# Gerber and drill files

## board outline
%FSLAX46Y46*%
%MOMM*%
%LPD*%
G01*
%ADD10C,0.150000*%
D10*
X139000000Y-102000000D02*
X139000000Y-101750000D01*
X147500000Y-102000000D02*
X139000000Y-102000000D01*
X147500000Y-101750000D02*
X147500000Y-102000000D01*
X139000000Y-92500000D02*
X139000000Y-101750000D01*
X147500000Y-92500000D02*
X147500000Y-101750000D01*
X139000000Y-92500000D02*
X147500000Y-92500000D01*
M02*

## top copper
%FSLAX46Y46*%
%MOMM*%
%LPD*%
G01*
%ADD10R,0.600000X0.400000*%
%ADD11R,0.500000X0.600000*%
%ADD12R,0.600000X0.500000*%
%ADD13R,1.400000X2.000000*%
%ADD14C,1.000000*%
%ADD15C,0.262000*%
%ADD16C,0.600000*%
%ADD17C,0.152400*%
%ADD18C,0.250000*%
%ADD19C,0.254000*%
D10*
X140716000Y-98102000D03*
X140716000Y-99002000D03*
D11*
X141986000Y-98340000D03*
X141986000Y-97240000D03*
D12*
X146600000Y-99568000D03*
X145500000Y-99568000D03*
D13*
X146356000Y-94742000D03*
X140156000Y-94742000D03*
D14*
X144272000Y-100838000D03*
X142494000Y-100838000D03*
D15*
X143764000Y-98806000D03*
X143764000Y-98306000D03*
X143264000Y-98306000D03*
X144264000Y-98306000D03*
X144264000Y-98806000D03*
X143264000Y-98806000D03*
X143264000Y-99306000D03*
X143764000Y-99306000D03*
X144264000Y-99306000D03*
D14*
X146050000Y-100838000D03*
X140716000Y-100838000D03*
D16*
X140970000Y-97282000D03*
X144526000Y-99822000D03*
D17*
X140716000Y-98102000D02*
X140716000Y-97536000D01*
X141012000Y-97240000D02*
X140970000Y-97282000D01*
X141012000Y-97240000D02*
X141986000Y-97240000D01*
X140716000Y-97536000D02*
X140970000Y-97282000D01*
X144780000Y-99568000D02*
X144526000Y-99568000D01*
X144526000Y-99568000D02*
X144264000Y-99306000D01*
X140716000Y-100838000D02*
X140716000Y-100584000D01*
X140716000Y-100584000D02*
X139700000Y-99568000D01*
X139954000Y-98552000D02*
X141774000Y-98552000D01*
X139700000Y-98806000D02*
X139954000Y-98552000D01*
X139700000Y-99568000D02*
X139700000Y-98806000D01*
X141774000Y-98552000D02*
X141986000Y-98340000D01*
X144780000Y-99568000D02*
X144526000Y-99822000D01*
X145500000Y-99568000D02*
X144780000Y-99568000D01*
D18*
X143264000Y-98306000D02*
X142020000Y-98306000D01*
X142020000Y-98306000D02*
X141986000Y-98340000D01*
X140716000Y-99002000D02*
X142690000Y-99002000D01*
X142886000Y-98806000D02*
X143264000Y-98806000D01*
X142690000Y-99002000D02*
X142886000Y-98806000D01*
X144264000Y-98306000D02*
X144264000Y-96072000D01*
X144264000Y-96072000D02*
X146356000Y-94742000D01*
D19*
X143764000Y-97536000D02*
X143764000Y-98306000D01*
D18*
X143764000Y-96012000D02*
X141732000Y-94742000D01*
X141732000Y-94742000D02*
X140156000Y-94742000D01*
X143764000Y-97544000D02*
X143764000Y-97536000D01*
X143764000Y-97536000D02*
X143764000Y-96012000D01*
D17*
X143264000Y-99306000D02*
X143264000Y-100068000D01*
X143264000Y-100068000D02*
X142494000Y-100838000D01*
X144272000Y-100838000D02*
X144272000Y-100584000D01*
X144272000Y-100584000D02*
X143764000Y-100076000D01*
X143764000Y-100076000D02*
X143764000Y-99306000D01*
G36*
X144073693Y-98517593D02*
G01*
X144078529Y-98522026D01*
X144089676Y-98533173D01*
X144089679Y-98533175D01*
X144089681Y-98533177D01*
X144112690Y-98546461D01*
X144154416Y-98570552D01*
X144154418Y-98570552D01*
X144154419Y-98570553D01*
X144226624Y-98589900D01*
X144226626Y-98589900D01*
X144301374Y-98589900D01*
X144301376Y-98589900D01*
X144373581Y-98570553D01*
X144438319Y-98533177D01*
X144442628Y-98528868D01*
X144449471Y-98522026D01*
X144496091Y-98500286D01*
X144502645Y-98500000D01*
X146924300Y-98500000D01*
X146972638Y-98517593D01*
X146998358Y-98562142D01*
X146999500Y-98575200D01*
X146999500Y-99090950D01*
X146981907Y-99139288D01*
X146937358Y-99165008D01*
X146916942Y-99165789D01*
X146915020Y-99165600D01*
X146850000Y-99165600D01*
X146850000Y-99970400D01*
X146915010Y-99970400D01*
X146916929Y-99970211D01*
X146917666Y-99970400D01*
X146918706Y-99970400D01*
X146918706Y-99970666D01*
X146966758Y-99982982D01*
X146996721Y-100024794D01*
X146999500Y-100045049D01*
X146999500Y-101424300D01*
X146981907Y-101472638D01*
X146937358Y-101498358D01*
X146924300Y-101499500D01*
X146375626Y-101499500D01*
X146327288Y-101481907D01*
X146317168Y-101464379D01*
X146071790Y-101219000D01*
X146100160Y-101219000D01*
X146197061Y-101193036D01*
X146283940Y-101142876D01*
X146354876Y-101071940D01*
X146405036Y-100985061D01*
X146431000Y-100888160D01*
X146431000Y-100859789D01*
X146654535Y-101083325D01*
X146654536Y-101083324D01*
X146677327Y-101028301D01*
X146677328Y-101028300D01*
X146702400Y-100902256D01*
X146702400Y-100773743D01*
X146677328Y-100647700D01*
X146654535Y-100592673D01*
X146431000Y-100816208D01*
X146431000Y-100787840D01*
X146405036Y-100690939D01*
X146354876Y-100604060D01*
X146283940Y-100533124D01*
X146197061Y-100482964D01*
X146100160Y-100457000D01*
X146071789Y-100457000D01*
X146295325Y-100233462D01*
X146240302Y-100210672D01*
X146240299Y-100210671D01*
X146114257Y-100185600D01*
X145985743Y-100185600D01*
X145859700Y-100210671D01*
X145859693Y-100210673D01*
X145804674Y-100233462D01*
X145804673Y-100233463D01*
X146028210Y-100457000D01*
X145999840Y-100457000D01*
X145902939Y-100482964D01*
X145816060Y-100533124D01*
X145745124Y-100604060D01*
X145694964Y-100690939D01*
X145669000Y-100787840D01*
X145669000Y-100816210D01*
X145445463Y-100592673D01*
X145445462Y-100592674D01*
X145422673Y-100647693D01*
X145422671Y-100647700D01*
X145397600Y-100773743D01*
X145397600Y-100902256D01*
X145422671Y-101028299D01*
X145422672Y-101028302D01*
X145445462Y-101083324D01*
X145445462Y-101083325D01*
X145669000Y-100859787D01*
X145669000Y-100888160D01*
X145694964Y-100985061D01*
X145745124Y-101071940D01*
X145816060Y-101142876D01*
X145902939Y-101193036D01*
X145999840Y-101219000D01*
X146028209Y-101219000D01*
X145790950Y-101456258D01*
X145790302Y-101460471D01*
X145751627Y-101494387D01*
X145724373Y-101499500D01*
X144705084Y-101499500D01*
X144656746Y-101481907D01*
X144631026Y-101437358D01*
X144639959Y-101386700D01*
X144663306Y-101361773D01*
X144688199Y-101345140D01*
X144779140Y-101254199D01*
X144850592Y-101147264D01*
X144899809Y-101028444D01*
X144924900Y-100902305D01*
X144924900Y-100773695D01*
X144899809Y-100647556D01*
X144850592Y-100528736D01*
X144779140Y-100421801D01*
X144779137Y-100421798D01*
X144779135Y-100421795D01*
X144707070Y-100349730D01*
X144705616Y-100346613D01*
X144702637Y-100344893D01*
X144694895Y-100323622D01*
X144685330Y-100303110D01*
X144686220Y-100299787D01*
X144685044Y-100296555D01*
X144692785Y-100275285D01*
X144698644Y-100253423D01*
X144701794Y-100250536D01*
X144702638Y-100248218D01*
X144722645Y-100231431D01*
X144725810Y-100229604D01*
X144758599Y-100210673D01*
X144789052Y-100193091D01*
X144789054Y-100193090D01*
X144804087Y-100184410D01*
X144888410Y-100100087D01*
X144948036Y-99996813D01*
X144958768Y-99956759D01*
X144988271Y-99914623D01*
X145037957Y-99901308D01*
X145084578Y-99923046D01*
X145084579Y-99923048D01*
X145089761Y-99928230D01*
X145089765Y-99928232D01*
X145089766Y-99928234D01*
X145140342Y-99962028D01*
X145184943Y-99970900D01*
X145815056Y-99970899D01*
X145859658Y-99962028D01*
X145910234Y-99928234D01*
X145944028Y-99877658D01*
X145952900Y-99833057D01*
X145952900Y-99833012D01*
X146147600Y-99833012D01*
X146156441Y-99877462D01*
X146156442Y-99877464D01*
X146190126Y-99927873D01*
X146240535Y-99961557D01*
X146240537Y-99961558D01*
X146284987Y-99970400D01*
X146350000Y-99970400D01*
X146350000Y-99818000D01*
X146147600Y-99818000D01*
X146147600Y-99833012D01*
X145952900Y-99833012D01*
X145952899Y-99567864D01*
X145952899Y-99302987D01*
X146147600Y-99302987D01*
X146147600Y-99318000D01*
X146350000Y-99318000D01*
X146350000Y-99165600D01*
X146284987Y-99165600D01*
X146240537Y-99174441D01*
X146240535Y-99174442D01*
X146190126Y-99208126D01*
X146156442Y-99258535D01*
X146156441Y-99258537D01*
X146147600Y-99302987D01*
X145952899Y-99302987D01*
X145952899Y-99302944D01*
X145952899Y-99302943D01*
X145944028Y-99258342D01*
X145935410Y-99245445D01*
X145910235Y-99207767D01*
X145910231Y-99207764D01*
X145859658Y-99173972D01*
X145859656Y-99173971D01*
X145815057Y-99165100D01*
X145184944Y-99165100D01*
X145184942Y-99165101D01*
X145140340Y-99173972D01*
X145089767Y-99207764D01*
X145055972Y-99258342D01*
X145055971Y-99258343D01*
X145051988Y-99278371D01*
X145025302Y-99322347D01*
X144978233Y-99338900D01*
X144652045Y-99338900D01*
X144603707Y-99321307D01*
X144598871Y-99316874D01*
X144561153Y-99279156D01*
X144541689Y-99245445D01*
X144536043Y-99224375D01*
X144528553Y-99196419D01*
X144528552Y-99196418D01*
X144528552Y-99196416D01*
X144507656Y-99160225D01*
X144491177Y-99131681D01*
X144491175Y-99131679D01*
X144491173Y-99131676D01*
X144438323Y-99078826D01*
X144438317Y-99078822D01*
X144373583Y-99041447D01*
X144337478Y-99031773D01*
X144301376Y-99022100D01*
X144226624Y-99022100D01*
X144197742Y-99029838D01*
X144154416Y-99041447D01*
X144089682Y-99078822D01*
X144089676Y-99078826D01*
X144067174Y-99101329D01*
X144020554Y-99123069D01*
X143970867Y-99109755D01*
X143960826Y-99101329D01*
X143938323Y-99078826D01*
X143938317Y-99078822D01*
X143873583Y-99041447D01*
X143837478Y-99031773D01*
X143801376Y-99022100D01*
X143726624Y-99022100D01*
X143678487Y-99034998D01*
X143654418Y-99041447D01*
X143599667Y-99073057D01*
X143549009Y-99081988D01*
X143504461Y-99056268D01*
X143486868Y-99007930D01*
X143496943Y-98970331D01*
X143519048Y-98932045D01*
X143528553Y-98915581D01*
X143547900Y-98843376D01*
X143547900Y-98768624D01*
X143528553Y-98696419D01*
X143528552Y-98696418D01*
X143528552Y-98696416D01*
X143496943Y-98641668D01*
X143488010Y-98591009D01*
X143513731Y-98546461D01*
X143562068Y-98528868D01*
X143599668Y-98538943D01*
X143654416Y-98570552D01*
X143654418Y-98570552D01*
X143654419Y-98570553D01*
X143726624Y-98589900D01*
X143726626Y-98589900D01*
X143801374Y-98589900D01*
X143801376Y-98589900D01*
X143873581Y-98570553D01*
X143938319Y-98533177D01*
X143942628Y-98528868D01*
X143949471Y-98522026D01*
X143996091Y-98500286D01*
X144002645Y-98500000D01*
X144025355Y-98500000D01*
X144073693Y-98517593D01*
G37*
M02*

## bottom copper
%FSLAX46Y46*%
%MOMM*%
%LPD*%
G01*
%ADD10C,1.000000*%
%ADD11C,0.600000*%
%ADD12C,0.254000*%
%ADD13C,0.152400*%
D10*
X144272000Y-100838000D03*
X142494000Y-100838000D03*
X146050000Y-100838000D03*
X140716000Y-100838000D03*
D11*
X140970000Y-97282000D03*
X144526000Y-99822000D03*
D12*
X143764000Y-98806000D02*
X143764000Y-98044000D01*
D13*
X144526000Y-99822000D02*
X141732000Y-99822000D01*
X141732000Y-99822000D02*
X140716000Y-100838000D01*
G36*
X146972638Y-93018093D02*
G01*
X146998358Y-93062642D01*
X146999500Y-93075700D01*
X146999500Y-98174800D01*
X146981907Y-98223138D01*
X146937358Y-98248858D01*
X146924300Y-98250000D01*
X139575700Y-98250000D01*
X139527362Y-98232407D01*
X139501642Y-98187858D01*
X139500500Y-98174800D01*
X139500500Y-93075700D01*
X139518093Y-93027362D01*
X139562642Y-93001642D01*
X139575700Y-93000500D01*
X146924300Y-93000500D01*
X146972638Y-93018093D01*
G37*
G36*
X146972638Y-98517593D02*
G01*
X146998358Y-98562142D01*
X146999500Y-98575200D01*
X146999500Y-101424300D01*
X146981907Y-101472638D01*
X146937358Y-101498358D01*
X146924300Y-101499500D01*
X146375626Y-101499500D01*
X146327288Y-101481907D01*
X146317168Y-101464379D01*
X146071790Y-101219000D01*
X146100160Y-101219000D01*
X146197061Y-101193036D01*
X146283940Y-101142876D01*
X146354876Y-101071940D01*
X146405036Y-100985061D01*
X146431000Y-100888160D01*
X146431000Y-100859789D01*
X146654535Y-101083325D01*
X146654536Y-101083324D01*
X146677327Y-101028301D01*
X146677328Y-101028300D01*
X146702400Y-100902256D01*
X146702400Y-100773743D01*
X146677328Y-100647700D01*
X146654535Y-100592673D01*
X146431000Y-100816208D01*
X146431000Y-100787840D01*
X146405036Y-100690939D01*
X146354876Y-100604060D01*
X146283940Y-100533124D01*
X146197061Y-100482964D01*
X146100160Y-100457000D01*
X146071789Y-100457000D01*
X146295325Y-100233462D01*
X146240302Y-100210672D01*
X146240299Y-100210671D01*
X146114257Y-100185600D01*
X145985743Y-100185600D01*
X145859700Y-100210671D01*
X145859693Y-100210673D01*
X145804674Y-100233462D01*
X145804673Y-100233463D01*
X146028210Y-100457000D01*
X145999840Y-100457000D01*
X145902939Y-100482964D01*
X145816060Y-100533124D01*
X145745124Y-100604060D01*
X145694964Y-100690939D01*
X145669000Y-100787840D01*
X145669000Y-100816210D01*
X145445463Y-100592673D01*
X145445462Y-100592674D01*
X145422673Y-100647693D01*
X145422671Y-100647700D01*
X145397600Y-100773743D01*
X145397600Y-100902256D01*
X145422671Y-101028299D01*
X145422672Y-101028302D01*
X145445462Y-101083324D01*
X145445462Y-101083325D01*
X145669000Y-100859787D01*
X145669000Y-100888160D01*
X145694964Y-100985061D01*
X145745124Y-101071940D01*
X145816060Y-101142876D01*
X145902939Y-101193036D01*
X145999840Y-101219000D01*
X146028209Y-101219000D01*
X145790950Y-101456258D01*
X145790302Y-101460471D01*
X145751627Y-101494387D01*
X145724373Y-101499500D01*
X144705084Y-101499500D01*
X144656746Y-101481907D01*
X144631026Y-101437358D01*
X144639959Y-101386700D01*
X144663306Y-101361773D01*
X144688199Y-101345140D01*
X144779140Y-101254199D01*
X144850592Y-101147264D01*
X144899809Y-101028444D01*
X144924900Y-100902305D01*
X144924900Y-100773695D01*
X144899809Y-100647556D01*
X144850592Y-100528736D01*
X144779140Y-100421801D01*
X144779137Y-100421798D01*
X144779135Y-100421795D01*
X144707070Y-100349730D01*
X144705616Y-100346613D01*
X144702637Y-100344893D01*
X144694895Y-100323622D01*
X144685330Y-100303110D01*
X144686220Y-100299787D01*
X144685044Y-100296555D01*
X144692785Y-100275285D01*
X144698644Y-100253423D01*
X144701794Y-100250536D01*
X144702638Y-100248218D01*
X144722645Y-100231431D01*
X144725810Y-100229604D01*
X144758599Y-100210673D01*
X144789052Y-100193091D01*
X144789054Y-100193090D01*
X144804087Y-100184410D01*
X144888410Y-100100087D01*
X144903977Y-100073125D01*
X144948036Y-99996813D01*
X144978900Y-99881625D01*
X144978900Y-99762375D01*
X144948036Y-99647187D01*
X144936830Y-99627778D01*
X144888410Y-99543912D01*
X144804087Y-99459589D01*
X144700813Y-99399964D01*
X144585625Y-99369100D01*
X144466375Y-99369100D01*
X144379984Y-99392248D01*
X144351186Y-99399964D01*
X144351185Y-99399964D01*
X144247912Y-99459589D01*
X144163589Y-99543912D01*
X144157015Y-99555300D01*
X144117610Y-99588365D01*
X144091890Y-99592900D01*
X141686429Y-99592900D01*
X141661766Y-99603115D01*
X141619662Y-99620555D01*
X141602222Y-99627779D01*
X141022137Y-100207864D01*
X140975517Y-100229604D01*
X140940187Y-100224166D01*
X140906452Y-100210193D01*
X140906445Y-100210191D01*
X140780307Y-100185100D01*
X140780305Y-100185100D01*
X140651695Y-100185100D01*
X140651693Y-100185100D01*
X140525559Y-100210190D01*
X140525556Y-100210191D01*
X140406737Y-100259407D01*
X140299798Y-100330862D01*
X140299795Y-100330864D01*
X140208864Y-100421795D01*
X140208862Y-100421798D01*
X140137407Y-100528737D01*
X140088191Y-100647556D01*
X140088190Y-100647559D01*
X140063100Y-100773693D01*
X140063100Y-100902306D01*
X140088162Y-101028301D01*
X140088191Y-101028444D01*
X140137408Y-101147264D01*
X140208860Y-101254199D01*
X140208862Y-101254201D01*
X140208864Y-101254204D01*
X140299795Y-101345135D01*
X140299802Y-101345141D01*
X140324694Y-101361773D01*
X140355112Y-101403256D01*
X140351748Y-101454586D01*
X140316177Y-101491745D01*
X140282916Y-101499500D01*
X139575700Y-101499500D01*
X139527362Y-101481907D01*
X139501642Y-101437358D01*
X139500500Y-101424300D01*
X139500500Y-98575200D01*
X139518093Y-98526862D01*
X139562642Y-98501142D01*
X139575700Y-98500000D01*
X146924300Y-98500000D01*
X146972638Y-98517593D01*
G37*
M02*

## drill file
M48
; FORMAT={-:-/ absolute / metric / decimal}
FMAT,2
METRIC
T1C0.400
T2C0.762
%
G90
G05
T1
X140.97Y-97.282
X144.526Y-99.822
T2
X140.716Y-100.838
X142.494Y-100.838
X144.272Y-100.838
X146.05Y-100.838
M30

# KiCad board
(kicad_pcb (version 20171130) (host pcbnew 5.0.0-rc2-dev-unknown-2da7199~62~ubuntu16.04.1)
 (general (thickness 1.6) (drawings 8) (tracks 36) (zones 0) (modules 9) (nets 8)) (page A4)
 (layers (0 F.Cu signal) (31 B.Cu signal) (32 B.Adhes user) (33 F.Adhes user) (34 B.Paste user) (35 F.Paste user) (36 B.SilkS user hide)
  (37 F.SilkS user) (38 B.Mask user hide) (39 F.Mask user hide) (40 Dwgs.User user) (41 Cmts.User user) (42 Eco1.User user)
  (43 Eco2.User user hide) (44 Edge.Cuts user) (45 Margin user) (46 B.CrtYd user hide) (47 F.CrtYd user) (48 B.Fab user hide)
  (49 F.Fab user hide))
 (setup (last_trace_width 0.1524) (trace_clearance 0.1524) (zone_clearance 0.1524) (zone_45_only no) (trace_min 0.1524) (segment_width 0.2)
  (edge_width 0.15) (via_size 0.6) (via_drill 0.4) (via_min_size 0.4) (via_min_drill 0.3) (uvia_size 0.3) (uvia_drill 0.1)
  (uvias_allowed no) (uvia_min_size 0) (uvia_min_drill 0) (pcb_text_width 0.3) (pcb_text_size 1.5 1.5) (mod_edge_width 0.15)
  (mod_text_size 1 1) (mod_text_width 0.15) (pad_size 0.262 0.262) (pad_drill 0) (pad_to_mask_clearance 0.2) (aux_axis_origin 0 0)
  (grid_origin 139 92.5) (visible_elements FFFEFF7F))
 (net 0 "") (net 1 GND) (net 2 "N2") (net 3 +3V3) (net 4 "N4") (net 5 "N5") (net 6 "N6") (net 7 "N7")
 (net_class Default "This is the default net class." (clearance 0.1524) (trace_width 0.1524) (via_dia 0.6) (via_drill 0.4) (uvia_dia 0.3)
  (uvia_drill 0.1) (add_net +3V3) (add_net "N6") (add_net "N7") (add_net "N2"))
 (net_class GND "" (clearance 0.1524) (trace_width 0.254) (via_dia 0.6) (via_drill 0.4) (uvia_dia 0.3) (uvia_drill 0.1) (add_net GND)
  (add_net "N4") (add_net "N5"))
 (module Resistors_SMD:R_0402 (layer F.Cu) (at 140.716 98.552 270)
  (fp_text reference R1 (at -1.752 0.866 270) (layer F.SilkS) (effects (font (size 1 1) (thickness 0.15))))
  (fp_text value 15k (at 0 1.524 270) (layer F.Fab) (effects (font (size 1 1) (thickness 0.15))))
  (pad 1 smd rect (at -0.45 0 270) (size 0.4 0.6) (layers F.Cu F.Paste F.Mask) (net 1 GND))
  (pad 2 smd rect (at 0.45 0 270) (size 0.4 0.6) (layers F.Cu F.Paste F.Mask) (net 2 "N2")))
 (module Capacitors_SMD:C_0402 (layer F.Cu) (at 141.986 97.79 90)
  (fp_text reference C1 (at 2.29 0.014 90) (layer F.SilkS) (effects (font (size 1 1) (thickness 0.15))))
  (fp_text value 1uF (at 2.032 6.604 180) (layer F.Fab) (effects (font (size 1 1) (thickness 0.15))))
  (pad 1 smd rect (at -0.55 0 90) (size 0.6 0.5) (layers F.Cu F.Paste F.Mask) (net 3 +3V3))
  (pad 2 smd rect (at 0.55 0 90) (size 0.6 0.5) (layers F.Cu F.Paste F.Mask) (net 1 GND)))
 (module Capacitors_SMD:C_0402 (layer F.Cu) (at 146.05 99.568 180)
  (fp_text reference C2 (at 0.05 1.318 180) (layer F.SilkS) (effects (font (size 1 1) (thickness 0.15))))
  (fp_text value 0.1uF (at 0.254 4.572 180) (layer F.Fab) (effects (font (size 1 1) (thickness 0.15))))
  (pad 1 smd rect (at -0.55 0 180) (size 0.6 0.5) (layers F.Cu F.Paste F.Mask) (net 1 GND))
  (pad 2 smd rect (at 0.55 0 180) (size 0.6 0.5) (layers F.Cu F.Paste F.Mask) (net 3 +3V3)))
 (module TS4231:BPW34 (layer F.Cu) (at 143.256 94.742 180)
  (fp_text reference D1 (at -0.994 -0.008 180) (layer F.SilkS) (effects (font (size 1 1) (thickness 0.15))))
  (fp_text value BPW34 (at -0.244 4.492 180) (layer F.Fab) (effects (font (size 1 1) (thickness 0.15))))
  (pad 1 smd rect (at -3.1 0 180) (size 1.4 2) (layers F.Cu F.Paste F.Mask) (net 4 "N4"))
  (pad 2 smd rect (at 3.1 0 180) (size 1.4 2) (layers F.Cu F.Paste F.Mask) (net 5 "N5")))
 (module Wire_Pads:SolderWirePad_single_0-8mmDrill (layer F.Cu) (at 144.272 100.838)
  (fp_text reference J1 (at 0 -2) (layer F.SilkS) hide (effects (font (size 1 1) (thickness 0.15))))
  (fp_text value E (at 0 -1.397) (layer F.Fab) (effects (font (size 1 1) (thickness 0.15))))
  (pad 1 thru_hole circle (at 0 0) (size 1 1) (drill 0.762) (layers *.Cu *.Mask F.SilkS) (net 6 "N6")))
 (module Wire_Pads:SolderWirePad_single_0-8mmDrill (layer F.Cu) (at 142.494 100.838)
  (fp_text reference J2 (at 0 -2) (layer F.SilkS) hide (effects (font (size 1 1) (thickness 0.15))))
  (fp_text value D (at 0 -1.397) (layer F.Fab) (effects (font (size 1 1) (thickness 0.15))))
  (pad 1 thru_hole circle (at 0 0) (size 1 1) (drill 0.762) (layers *.Cu *.Mask F.SilkS) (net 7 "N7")))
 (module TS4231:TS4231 (layer F.Cu) (at 143.764 98.806)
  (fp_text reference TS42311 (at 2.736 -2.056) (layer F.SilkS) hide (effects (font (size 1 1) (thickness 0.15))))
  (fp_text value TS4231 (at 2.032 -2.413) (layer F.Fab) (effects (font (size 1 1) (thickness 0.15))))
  (pad 5 smd circle (at 0 0) (size 0.262 0.262) (layers F.Cu F.Paste F.Mask) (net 1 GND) (zone_connect 2))
  (pad 2 smd circle (at 0 -0.5) (size 0.262 0.262) (layers F.Cu F.Paste F.Mask) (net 5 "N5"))
  (pad 1 smd circle (at -0.5 -0.5) (size 0.262 0.262) (layers F.Cu F.Paste F.Mask) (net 3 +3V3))
  (pad 3 smd circle (at 0.5 -0.5) (size 0.262 0.262) (layers F.Cu F.Paste F.Mask) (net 4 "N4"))
  (pad 6 smd circle (at 0.5 0) (size 0.262 0.262) (layers F.Cu F.Paste F.Mask) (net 1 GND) (zone_connect 2))
  (pad 4 smd circle (at -0.5 0) (size 0.262 0.262) (layers F.Cu F.Paste F.Mask) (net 2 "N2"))
  (pad 7 smd circle (at -0.5 0.5) (size 0.262 0.262) (layers F.Cu F.Paste F.Mask) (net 7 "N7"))
  (pad 8 smd circle (at 0 0.5) (size 0.262 0.262) (layers F.Cu F.Paste F.Mask) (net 6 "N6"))
  (pad 9 smd circle (at 0.5 0.5) (size 0.262 0.262) (layers F.Cu F.Paste F.Mask) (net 3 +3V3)))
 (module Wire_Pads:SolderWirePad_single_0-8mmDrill (layer F.Cu) (at 146.05 100.838)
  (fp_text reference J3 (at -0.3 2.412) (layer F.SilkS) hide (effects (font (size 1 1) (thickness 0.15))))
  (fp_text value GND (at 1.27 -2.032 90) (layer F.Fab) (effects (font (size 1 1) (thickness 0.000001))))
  (pad 1 thru_hole circle (at 0 0) (size 1 1) (drill 0.762) (layers *.Cu *.Mask F.SilkS) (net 1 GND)))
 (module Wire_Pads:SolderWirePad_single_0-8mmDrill (layer F.Cu) (at 140.716 100.838)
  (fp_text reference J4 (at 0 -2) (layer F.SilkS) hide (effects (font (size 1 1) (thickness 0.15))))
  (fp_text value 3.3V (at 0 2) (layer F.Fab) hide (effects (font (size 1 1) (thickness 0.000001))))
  (pad 1 thru_hole circle (at 0 0) (size 1 1) (drill 0.762) (layers *.Cu *.Mask F.SilkS) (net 3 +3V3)))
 (gr_line (start 139 102) (end 139 101.75) (angle 90) (layer Edge.Cuts) (width 0.15))
 (gr_line (start 147.5 102) (end 139 102) (angle 90) (layer Edge.Cuts) (width 0.15))
 (gr_line (start 147.5 101.75) (end 147.5 102) (angle 90) (layer Edge.Cuts) (width 0.15))
 (gr_line (start 139 92.5) (end 139 101.75) (angle 90) (layer Edge.Cuts) (width 0.15))
 (gr_line (start 147.5 92.5) (end 147.5 101.75) (angle 90) (layer Edge.Cuts) (width 0.15))
 (gr_line (start 139 92.5) (end 147.5 92.5) (angle 90) (layer Edge.Cuts) (width 0.15))
 (segment (start 143.764 98.806) (end 143.764 98.044) (width 0.254) (layer B.Cu) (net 1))
 (segment (start 140.716 98.102) (end 140.716 97.536) (width 0.1524) (layer F.Cu) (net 1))
 (segment (start 141.012 97.24) (end 140.97 97.282) (width 0.1524) (layer F.Cu) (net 1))
 (via (at 140.97 97.282) (size 0.6) (drill 0.4) (layers F.Cu B.Cu) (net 1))
 (segment (start 141.012 97.24) (end 141.986 97.24) (width 0.1524) (layer F.Cu) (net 1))
 (segment (start 140.716 97.536) (end 140.97 97.282) (width 0.1524) (layer F.Cu) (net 1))
 (segment (start 144.78 99.568) (end 144.526 99.568) (width 0.1524) (layer F.Cu) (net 3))
 (segment (start 144.526 99.568) (end 144.264 99.306) (width 0.1524) (layer F.Cu) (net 3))
 (segment (start 140.716 100.838) (end 140.716 100.584) (width 0.1524) (layer F.Cu) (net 3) (status C00000))
 (segment (start 140.716 100.584) (end 139.7 99.568) (width 0.1524) (layer F.Cu) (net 3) (status 400000))
 (segment (start 139.954 98.552) (end 141.774 98.552) (width 0.1524) (layer F.Cu) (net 3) (status 800000))
 (segment (start 139.7 98.806) (end 139.954 98.552) (width 0.1524) (layer F.Cu) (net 3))
 (segment (start 139.7 99.568) (end 139.7 98.806) (width 0.1524) (layer F.Cu) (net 3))
 (segment (start 141.774 98.552) (end 141.986 98.34) (width 0.1524) (layer F.Cu) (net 3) (status C00000))
 (segment (start 144.526 99.822) (end 141.732 99.822) (width 0.1524) (layer B.Cu) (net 3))
 (segment (start 144.78 99.568) (end 144.526 99.822) (width 0.1524) (layer F.Cu) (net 3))
 (via (at 144.526 99.822) (size 0.6) (drill 0.4) (layers F.Cu B.Cu) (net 3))
 (segment (start 145.5 99.568) (end 144.78 99.568) (width 0.1524) (layer F.Cu) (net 3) (status 400000))
 (segment (start 141.732 99.822) (end 140.716 100.838) (width 0.1524) (layer B.Cu) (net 3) (status 800000))
 (segment (start 143.264 98.306) (end 142.02 98.306) (width 0.25) (layer F.Cu) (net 3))
 (segment (start 142.02 98.306) (end 141.986 98.34) (width 0.25) (layer F.Cu) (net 3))
 (segment (start 140.716 99.002) (end 142.69 99.002) (width 0.25) (layer F.Cu) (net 2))
 (segment (start 142.886 98.806) (end 143.264 98.806) (width 0.25) (layer F.Cu) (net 2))
 (segment (start 142.69 99.002) (end 142.886 98.806) (width 0.25) (layer F.Cu) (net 2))
 (segment (start 144.264 98.306) (end 144.264 96.072) (width 0.25) (layer F.Cu) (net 4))
 (segment (start 144.264 96.072) (end 146.356 94.742) (width 0.25) (layer F.Cu) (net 4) (status 20))
 (segment (start 143.764 97.536) (end 143.764 98.306) (width 0.254) (layer F.Cu) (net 5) (status 800000))
 (segment (start 143.764 96.012) (end 141.732 94.742) (width 0.25) (layer F.Cu) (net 5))
 (segment (start 141.732 94.742) (end 140.156 94.742) (width 0.25) (layer F.Cu) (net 5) (status 20))
 (segment (start 143.764 97.544) (end 143.764 97.536) (width 0.25) (layer F.Cu) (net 5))
 (segment (start 143.764 97.536) (end 143.764 96.012) (width 0.25) (layer F.Cu) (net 5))
 (segment (start 143.264 99.306) (end 143.264 100.068) (width 0.1524) (layer F.Cu) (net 7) (status 400000))
 (segment (start 143.264 100.068) (end 142.494 100.838) (width 0.1524) (layer F.Cu) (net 7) (status 800000))
 (segment (start 144.272 100.838) (end 144.272 100.584) (width 0.1524) (layer F.Cu) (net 6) (status C00000))
 (segment (start 144.272 100.584) (end 143.764 100.076) (width 0.1524) (layer F.Cu) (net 6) (status 400000))
 (segment (start 143.764 100.076) (end 143.764 99.306) (width 0.1524) (layer F.Cu) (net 6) (status 800000))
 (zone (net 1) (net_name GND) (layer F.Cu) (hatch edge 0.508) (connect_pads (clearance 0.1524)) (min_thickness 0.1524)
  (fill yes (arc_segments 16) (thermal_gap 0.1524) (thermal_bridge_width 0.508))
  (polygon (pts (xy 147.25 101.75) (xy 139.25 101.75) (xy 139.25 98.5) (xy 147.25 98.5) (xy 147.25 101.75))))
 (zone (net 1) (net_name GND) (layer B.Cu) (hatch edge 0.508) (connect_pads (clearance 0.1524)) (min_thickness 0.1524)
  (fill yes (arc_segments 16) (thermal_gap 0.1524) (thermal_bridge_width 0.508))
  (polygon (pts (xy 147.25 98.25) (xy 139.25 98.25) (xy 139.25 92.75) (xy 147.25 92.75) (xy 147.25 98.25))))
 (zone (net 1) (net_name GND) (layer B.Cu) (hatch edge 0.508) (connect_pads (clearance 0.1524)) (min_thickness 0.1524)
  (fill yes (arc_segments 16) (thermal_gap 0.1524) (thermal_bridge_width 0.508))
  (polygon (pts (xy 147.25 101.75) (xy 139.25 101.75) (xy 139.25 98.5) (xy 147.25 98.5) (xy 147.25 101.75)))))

